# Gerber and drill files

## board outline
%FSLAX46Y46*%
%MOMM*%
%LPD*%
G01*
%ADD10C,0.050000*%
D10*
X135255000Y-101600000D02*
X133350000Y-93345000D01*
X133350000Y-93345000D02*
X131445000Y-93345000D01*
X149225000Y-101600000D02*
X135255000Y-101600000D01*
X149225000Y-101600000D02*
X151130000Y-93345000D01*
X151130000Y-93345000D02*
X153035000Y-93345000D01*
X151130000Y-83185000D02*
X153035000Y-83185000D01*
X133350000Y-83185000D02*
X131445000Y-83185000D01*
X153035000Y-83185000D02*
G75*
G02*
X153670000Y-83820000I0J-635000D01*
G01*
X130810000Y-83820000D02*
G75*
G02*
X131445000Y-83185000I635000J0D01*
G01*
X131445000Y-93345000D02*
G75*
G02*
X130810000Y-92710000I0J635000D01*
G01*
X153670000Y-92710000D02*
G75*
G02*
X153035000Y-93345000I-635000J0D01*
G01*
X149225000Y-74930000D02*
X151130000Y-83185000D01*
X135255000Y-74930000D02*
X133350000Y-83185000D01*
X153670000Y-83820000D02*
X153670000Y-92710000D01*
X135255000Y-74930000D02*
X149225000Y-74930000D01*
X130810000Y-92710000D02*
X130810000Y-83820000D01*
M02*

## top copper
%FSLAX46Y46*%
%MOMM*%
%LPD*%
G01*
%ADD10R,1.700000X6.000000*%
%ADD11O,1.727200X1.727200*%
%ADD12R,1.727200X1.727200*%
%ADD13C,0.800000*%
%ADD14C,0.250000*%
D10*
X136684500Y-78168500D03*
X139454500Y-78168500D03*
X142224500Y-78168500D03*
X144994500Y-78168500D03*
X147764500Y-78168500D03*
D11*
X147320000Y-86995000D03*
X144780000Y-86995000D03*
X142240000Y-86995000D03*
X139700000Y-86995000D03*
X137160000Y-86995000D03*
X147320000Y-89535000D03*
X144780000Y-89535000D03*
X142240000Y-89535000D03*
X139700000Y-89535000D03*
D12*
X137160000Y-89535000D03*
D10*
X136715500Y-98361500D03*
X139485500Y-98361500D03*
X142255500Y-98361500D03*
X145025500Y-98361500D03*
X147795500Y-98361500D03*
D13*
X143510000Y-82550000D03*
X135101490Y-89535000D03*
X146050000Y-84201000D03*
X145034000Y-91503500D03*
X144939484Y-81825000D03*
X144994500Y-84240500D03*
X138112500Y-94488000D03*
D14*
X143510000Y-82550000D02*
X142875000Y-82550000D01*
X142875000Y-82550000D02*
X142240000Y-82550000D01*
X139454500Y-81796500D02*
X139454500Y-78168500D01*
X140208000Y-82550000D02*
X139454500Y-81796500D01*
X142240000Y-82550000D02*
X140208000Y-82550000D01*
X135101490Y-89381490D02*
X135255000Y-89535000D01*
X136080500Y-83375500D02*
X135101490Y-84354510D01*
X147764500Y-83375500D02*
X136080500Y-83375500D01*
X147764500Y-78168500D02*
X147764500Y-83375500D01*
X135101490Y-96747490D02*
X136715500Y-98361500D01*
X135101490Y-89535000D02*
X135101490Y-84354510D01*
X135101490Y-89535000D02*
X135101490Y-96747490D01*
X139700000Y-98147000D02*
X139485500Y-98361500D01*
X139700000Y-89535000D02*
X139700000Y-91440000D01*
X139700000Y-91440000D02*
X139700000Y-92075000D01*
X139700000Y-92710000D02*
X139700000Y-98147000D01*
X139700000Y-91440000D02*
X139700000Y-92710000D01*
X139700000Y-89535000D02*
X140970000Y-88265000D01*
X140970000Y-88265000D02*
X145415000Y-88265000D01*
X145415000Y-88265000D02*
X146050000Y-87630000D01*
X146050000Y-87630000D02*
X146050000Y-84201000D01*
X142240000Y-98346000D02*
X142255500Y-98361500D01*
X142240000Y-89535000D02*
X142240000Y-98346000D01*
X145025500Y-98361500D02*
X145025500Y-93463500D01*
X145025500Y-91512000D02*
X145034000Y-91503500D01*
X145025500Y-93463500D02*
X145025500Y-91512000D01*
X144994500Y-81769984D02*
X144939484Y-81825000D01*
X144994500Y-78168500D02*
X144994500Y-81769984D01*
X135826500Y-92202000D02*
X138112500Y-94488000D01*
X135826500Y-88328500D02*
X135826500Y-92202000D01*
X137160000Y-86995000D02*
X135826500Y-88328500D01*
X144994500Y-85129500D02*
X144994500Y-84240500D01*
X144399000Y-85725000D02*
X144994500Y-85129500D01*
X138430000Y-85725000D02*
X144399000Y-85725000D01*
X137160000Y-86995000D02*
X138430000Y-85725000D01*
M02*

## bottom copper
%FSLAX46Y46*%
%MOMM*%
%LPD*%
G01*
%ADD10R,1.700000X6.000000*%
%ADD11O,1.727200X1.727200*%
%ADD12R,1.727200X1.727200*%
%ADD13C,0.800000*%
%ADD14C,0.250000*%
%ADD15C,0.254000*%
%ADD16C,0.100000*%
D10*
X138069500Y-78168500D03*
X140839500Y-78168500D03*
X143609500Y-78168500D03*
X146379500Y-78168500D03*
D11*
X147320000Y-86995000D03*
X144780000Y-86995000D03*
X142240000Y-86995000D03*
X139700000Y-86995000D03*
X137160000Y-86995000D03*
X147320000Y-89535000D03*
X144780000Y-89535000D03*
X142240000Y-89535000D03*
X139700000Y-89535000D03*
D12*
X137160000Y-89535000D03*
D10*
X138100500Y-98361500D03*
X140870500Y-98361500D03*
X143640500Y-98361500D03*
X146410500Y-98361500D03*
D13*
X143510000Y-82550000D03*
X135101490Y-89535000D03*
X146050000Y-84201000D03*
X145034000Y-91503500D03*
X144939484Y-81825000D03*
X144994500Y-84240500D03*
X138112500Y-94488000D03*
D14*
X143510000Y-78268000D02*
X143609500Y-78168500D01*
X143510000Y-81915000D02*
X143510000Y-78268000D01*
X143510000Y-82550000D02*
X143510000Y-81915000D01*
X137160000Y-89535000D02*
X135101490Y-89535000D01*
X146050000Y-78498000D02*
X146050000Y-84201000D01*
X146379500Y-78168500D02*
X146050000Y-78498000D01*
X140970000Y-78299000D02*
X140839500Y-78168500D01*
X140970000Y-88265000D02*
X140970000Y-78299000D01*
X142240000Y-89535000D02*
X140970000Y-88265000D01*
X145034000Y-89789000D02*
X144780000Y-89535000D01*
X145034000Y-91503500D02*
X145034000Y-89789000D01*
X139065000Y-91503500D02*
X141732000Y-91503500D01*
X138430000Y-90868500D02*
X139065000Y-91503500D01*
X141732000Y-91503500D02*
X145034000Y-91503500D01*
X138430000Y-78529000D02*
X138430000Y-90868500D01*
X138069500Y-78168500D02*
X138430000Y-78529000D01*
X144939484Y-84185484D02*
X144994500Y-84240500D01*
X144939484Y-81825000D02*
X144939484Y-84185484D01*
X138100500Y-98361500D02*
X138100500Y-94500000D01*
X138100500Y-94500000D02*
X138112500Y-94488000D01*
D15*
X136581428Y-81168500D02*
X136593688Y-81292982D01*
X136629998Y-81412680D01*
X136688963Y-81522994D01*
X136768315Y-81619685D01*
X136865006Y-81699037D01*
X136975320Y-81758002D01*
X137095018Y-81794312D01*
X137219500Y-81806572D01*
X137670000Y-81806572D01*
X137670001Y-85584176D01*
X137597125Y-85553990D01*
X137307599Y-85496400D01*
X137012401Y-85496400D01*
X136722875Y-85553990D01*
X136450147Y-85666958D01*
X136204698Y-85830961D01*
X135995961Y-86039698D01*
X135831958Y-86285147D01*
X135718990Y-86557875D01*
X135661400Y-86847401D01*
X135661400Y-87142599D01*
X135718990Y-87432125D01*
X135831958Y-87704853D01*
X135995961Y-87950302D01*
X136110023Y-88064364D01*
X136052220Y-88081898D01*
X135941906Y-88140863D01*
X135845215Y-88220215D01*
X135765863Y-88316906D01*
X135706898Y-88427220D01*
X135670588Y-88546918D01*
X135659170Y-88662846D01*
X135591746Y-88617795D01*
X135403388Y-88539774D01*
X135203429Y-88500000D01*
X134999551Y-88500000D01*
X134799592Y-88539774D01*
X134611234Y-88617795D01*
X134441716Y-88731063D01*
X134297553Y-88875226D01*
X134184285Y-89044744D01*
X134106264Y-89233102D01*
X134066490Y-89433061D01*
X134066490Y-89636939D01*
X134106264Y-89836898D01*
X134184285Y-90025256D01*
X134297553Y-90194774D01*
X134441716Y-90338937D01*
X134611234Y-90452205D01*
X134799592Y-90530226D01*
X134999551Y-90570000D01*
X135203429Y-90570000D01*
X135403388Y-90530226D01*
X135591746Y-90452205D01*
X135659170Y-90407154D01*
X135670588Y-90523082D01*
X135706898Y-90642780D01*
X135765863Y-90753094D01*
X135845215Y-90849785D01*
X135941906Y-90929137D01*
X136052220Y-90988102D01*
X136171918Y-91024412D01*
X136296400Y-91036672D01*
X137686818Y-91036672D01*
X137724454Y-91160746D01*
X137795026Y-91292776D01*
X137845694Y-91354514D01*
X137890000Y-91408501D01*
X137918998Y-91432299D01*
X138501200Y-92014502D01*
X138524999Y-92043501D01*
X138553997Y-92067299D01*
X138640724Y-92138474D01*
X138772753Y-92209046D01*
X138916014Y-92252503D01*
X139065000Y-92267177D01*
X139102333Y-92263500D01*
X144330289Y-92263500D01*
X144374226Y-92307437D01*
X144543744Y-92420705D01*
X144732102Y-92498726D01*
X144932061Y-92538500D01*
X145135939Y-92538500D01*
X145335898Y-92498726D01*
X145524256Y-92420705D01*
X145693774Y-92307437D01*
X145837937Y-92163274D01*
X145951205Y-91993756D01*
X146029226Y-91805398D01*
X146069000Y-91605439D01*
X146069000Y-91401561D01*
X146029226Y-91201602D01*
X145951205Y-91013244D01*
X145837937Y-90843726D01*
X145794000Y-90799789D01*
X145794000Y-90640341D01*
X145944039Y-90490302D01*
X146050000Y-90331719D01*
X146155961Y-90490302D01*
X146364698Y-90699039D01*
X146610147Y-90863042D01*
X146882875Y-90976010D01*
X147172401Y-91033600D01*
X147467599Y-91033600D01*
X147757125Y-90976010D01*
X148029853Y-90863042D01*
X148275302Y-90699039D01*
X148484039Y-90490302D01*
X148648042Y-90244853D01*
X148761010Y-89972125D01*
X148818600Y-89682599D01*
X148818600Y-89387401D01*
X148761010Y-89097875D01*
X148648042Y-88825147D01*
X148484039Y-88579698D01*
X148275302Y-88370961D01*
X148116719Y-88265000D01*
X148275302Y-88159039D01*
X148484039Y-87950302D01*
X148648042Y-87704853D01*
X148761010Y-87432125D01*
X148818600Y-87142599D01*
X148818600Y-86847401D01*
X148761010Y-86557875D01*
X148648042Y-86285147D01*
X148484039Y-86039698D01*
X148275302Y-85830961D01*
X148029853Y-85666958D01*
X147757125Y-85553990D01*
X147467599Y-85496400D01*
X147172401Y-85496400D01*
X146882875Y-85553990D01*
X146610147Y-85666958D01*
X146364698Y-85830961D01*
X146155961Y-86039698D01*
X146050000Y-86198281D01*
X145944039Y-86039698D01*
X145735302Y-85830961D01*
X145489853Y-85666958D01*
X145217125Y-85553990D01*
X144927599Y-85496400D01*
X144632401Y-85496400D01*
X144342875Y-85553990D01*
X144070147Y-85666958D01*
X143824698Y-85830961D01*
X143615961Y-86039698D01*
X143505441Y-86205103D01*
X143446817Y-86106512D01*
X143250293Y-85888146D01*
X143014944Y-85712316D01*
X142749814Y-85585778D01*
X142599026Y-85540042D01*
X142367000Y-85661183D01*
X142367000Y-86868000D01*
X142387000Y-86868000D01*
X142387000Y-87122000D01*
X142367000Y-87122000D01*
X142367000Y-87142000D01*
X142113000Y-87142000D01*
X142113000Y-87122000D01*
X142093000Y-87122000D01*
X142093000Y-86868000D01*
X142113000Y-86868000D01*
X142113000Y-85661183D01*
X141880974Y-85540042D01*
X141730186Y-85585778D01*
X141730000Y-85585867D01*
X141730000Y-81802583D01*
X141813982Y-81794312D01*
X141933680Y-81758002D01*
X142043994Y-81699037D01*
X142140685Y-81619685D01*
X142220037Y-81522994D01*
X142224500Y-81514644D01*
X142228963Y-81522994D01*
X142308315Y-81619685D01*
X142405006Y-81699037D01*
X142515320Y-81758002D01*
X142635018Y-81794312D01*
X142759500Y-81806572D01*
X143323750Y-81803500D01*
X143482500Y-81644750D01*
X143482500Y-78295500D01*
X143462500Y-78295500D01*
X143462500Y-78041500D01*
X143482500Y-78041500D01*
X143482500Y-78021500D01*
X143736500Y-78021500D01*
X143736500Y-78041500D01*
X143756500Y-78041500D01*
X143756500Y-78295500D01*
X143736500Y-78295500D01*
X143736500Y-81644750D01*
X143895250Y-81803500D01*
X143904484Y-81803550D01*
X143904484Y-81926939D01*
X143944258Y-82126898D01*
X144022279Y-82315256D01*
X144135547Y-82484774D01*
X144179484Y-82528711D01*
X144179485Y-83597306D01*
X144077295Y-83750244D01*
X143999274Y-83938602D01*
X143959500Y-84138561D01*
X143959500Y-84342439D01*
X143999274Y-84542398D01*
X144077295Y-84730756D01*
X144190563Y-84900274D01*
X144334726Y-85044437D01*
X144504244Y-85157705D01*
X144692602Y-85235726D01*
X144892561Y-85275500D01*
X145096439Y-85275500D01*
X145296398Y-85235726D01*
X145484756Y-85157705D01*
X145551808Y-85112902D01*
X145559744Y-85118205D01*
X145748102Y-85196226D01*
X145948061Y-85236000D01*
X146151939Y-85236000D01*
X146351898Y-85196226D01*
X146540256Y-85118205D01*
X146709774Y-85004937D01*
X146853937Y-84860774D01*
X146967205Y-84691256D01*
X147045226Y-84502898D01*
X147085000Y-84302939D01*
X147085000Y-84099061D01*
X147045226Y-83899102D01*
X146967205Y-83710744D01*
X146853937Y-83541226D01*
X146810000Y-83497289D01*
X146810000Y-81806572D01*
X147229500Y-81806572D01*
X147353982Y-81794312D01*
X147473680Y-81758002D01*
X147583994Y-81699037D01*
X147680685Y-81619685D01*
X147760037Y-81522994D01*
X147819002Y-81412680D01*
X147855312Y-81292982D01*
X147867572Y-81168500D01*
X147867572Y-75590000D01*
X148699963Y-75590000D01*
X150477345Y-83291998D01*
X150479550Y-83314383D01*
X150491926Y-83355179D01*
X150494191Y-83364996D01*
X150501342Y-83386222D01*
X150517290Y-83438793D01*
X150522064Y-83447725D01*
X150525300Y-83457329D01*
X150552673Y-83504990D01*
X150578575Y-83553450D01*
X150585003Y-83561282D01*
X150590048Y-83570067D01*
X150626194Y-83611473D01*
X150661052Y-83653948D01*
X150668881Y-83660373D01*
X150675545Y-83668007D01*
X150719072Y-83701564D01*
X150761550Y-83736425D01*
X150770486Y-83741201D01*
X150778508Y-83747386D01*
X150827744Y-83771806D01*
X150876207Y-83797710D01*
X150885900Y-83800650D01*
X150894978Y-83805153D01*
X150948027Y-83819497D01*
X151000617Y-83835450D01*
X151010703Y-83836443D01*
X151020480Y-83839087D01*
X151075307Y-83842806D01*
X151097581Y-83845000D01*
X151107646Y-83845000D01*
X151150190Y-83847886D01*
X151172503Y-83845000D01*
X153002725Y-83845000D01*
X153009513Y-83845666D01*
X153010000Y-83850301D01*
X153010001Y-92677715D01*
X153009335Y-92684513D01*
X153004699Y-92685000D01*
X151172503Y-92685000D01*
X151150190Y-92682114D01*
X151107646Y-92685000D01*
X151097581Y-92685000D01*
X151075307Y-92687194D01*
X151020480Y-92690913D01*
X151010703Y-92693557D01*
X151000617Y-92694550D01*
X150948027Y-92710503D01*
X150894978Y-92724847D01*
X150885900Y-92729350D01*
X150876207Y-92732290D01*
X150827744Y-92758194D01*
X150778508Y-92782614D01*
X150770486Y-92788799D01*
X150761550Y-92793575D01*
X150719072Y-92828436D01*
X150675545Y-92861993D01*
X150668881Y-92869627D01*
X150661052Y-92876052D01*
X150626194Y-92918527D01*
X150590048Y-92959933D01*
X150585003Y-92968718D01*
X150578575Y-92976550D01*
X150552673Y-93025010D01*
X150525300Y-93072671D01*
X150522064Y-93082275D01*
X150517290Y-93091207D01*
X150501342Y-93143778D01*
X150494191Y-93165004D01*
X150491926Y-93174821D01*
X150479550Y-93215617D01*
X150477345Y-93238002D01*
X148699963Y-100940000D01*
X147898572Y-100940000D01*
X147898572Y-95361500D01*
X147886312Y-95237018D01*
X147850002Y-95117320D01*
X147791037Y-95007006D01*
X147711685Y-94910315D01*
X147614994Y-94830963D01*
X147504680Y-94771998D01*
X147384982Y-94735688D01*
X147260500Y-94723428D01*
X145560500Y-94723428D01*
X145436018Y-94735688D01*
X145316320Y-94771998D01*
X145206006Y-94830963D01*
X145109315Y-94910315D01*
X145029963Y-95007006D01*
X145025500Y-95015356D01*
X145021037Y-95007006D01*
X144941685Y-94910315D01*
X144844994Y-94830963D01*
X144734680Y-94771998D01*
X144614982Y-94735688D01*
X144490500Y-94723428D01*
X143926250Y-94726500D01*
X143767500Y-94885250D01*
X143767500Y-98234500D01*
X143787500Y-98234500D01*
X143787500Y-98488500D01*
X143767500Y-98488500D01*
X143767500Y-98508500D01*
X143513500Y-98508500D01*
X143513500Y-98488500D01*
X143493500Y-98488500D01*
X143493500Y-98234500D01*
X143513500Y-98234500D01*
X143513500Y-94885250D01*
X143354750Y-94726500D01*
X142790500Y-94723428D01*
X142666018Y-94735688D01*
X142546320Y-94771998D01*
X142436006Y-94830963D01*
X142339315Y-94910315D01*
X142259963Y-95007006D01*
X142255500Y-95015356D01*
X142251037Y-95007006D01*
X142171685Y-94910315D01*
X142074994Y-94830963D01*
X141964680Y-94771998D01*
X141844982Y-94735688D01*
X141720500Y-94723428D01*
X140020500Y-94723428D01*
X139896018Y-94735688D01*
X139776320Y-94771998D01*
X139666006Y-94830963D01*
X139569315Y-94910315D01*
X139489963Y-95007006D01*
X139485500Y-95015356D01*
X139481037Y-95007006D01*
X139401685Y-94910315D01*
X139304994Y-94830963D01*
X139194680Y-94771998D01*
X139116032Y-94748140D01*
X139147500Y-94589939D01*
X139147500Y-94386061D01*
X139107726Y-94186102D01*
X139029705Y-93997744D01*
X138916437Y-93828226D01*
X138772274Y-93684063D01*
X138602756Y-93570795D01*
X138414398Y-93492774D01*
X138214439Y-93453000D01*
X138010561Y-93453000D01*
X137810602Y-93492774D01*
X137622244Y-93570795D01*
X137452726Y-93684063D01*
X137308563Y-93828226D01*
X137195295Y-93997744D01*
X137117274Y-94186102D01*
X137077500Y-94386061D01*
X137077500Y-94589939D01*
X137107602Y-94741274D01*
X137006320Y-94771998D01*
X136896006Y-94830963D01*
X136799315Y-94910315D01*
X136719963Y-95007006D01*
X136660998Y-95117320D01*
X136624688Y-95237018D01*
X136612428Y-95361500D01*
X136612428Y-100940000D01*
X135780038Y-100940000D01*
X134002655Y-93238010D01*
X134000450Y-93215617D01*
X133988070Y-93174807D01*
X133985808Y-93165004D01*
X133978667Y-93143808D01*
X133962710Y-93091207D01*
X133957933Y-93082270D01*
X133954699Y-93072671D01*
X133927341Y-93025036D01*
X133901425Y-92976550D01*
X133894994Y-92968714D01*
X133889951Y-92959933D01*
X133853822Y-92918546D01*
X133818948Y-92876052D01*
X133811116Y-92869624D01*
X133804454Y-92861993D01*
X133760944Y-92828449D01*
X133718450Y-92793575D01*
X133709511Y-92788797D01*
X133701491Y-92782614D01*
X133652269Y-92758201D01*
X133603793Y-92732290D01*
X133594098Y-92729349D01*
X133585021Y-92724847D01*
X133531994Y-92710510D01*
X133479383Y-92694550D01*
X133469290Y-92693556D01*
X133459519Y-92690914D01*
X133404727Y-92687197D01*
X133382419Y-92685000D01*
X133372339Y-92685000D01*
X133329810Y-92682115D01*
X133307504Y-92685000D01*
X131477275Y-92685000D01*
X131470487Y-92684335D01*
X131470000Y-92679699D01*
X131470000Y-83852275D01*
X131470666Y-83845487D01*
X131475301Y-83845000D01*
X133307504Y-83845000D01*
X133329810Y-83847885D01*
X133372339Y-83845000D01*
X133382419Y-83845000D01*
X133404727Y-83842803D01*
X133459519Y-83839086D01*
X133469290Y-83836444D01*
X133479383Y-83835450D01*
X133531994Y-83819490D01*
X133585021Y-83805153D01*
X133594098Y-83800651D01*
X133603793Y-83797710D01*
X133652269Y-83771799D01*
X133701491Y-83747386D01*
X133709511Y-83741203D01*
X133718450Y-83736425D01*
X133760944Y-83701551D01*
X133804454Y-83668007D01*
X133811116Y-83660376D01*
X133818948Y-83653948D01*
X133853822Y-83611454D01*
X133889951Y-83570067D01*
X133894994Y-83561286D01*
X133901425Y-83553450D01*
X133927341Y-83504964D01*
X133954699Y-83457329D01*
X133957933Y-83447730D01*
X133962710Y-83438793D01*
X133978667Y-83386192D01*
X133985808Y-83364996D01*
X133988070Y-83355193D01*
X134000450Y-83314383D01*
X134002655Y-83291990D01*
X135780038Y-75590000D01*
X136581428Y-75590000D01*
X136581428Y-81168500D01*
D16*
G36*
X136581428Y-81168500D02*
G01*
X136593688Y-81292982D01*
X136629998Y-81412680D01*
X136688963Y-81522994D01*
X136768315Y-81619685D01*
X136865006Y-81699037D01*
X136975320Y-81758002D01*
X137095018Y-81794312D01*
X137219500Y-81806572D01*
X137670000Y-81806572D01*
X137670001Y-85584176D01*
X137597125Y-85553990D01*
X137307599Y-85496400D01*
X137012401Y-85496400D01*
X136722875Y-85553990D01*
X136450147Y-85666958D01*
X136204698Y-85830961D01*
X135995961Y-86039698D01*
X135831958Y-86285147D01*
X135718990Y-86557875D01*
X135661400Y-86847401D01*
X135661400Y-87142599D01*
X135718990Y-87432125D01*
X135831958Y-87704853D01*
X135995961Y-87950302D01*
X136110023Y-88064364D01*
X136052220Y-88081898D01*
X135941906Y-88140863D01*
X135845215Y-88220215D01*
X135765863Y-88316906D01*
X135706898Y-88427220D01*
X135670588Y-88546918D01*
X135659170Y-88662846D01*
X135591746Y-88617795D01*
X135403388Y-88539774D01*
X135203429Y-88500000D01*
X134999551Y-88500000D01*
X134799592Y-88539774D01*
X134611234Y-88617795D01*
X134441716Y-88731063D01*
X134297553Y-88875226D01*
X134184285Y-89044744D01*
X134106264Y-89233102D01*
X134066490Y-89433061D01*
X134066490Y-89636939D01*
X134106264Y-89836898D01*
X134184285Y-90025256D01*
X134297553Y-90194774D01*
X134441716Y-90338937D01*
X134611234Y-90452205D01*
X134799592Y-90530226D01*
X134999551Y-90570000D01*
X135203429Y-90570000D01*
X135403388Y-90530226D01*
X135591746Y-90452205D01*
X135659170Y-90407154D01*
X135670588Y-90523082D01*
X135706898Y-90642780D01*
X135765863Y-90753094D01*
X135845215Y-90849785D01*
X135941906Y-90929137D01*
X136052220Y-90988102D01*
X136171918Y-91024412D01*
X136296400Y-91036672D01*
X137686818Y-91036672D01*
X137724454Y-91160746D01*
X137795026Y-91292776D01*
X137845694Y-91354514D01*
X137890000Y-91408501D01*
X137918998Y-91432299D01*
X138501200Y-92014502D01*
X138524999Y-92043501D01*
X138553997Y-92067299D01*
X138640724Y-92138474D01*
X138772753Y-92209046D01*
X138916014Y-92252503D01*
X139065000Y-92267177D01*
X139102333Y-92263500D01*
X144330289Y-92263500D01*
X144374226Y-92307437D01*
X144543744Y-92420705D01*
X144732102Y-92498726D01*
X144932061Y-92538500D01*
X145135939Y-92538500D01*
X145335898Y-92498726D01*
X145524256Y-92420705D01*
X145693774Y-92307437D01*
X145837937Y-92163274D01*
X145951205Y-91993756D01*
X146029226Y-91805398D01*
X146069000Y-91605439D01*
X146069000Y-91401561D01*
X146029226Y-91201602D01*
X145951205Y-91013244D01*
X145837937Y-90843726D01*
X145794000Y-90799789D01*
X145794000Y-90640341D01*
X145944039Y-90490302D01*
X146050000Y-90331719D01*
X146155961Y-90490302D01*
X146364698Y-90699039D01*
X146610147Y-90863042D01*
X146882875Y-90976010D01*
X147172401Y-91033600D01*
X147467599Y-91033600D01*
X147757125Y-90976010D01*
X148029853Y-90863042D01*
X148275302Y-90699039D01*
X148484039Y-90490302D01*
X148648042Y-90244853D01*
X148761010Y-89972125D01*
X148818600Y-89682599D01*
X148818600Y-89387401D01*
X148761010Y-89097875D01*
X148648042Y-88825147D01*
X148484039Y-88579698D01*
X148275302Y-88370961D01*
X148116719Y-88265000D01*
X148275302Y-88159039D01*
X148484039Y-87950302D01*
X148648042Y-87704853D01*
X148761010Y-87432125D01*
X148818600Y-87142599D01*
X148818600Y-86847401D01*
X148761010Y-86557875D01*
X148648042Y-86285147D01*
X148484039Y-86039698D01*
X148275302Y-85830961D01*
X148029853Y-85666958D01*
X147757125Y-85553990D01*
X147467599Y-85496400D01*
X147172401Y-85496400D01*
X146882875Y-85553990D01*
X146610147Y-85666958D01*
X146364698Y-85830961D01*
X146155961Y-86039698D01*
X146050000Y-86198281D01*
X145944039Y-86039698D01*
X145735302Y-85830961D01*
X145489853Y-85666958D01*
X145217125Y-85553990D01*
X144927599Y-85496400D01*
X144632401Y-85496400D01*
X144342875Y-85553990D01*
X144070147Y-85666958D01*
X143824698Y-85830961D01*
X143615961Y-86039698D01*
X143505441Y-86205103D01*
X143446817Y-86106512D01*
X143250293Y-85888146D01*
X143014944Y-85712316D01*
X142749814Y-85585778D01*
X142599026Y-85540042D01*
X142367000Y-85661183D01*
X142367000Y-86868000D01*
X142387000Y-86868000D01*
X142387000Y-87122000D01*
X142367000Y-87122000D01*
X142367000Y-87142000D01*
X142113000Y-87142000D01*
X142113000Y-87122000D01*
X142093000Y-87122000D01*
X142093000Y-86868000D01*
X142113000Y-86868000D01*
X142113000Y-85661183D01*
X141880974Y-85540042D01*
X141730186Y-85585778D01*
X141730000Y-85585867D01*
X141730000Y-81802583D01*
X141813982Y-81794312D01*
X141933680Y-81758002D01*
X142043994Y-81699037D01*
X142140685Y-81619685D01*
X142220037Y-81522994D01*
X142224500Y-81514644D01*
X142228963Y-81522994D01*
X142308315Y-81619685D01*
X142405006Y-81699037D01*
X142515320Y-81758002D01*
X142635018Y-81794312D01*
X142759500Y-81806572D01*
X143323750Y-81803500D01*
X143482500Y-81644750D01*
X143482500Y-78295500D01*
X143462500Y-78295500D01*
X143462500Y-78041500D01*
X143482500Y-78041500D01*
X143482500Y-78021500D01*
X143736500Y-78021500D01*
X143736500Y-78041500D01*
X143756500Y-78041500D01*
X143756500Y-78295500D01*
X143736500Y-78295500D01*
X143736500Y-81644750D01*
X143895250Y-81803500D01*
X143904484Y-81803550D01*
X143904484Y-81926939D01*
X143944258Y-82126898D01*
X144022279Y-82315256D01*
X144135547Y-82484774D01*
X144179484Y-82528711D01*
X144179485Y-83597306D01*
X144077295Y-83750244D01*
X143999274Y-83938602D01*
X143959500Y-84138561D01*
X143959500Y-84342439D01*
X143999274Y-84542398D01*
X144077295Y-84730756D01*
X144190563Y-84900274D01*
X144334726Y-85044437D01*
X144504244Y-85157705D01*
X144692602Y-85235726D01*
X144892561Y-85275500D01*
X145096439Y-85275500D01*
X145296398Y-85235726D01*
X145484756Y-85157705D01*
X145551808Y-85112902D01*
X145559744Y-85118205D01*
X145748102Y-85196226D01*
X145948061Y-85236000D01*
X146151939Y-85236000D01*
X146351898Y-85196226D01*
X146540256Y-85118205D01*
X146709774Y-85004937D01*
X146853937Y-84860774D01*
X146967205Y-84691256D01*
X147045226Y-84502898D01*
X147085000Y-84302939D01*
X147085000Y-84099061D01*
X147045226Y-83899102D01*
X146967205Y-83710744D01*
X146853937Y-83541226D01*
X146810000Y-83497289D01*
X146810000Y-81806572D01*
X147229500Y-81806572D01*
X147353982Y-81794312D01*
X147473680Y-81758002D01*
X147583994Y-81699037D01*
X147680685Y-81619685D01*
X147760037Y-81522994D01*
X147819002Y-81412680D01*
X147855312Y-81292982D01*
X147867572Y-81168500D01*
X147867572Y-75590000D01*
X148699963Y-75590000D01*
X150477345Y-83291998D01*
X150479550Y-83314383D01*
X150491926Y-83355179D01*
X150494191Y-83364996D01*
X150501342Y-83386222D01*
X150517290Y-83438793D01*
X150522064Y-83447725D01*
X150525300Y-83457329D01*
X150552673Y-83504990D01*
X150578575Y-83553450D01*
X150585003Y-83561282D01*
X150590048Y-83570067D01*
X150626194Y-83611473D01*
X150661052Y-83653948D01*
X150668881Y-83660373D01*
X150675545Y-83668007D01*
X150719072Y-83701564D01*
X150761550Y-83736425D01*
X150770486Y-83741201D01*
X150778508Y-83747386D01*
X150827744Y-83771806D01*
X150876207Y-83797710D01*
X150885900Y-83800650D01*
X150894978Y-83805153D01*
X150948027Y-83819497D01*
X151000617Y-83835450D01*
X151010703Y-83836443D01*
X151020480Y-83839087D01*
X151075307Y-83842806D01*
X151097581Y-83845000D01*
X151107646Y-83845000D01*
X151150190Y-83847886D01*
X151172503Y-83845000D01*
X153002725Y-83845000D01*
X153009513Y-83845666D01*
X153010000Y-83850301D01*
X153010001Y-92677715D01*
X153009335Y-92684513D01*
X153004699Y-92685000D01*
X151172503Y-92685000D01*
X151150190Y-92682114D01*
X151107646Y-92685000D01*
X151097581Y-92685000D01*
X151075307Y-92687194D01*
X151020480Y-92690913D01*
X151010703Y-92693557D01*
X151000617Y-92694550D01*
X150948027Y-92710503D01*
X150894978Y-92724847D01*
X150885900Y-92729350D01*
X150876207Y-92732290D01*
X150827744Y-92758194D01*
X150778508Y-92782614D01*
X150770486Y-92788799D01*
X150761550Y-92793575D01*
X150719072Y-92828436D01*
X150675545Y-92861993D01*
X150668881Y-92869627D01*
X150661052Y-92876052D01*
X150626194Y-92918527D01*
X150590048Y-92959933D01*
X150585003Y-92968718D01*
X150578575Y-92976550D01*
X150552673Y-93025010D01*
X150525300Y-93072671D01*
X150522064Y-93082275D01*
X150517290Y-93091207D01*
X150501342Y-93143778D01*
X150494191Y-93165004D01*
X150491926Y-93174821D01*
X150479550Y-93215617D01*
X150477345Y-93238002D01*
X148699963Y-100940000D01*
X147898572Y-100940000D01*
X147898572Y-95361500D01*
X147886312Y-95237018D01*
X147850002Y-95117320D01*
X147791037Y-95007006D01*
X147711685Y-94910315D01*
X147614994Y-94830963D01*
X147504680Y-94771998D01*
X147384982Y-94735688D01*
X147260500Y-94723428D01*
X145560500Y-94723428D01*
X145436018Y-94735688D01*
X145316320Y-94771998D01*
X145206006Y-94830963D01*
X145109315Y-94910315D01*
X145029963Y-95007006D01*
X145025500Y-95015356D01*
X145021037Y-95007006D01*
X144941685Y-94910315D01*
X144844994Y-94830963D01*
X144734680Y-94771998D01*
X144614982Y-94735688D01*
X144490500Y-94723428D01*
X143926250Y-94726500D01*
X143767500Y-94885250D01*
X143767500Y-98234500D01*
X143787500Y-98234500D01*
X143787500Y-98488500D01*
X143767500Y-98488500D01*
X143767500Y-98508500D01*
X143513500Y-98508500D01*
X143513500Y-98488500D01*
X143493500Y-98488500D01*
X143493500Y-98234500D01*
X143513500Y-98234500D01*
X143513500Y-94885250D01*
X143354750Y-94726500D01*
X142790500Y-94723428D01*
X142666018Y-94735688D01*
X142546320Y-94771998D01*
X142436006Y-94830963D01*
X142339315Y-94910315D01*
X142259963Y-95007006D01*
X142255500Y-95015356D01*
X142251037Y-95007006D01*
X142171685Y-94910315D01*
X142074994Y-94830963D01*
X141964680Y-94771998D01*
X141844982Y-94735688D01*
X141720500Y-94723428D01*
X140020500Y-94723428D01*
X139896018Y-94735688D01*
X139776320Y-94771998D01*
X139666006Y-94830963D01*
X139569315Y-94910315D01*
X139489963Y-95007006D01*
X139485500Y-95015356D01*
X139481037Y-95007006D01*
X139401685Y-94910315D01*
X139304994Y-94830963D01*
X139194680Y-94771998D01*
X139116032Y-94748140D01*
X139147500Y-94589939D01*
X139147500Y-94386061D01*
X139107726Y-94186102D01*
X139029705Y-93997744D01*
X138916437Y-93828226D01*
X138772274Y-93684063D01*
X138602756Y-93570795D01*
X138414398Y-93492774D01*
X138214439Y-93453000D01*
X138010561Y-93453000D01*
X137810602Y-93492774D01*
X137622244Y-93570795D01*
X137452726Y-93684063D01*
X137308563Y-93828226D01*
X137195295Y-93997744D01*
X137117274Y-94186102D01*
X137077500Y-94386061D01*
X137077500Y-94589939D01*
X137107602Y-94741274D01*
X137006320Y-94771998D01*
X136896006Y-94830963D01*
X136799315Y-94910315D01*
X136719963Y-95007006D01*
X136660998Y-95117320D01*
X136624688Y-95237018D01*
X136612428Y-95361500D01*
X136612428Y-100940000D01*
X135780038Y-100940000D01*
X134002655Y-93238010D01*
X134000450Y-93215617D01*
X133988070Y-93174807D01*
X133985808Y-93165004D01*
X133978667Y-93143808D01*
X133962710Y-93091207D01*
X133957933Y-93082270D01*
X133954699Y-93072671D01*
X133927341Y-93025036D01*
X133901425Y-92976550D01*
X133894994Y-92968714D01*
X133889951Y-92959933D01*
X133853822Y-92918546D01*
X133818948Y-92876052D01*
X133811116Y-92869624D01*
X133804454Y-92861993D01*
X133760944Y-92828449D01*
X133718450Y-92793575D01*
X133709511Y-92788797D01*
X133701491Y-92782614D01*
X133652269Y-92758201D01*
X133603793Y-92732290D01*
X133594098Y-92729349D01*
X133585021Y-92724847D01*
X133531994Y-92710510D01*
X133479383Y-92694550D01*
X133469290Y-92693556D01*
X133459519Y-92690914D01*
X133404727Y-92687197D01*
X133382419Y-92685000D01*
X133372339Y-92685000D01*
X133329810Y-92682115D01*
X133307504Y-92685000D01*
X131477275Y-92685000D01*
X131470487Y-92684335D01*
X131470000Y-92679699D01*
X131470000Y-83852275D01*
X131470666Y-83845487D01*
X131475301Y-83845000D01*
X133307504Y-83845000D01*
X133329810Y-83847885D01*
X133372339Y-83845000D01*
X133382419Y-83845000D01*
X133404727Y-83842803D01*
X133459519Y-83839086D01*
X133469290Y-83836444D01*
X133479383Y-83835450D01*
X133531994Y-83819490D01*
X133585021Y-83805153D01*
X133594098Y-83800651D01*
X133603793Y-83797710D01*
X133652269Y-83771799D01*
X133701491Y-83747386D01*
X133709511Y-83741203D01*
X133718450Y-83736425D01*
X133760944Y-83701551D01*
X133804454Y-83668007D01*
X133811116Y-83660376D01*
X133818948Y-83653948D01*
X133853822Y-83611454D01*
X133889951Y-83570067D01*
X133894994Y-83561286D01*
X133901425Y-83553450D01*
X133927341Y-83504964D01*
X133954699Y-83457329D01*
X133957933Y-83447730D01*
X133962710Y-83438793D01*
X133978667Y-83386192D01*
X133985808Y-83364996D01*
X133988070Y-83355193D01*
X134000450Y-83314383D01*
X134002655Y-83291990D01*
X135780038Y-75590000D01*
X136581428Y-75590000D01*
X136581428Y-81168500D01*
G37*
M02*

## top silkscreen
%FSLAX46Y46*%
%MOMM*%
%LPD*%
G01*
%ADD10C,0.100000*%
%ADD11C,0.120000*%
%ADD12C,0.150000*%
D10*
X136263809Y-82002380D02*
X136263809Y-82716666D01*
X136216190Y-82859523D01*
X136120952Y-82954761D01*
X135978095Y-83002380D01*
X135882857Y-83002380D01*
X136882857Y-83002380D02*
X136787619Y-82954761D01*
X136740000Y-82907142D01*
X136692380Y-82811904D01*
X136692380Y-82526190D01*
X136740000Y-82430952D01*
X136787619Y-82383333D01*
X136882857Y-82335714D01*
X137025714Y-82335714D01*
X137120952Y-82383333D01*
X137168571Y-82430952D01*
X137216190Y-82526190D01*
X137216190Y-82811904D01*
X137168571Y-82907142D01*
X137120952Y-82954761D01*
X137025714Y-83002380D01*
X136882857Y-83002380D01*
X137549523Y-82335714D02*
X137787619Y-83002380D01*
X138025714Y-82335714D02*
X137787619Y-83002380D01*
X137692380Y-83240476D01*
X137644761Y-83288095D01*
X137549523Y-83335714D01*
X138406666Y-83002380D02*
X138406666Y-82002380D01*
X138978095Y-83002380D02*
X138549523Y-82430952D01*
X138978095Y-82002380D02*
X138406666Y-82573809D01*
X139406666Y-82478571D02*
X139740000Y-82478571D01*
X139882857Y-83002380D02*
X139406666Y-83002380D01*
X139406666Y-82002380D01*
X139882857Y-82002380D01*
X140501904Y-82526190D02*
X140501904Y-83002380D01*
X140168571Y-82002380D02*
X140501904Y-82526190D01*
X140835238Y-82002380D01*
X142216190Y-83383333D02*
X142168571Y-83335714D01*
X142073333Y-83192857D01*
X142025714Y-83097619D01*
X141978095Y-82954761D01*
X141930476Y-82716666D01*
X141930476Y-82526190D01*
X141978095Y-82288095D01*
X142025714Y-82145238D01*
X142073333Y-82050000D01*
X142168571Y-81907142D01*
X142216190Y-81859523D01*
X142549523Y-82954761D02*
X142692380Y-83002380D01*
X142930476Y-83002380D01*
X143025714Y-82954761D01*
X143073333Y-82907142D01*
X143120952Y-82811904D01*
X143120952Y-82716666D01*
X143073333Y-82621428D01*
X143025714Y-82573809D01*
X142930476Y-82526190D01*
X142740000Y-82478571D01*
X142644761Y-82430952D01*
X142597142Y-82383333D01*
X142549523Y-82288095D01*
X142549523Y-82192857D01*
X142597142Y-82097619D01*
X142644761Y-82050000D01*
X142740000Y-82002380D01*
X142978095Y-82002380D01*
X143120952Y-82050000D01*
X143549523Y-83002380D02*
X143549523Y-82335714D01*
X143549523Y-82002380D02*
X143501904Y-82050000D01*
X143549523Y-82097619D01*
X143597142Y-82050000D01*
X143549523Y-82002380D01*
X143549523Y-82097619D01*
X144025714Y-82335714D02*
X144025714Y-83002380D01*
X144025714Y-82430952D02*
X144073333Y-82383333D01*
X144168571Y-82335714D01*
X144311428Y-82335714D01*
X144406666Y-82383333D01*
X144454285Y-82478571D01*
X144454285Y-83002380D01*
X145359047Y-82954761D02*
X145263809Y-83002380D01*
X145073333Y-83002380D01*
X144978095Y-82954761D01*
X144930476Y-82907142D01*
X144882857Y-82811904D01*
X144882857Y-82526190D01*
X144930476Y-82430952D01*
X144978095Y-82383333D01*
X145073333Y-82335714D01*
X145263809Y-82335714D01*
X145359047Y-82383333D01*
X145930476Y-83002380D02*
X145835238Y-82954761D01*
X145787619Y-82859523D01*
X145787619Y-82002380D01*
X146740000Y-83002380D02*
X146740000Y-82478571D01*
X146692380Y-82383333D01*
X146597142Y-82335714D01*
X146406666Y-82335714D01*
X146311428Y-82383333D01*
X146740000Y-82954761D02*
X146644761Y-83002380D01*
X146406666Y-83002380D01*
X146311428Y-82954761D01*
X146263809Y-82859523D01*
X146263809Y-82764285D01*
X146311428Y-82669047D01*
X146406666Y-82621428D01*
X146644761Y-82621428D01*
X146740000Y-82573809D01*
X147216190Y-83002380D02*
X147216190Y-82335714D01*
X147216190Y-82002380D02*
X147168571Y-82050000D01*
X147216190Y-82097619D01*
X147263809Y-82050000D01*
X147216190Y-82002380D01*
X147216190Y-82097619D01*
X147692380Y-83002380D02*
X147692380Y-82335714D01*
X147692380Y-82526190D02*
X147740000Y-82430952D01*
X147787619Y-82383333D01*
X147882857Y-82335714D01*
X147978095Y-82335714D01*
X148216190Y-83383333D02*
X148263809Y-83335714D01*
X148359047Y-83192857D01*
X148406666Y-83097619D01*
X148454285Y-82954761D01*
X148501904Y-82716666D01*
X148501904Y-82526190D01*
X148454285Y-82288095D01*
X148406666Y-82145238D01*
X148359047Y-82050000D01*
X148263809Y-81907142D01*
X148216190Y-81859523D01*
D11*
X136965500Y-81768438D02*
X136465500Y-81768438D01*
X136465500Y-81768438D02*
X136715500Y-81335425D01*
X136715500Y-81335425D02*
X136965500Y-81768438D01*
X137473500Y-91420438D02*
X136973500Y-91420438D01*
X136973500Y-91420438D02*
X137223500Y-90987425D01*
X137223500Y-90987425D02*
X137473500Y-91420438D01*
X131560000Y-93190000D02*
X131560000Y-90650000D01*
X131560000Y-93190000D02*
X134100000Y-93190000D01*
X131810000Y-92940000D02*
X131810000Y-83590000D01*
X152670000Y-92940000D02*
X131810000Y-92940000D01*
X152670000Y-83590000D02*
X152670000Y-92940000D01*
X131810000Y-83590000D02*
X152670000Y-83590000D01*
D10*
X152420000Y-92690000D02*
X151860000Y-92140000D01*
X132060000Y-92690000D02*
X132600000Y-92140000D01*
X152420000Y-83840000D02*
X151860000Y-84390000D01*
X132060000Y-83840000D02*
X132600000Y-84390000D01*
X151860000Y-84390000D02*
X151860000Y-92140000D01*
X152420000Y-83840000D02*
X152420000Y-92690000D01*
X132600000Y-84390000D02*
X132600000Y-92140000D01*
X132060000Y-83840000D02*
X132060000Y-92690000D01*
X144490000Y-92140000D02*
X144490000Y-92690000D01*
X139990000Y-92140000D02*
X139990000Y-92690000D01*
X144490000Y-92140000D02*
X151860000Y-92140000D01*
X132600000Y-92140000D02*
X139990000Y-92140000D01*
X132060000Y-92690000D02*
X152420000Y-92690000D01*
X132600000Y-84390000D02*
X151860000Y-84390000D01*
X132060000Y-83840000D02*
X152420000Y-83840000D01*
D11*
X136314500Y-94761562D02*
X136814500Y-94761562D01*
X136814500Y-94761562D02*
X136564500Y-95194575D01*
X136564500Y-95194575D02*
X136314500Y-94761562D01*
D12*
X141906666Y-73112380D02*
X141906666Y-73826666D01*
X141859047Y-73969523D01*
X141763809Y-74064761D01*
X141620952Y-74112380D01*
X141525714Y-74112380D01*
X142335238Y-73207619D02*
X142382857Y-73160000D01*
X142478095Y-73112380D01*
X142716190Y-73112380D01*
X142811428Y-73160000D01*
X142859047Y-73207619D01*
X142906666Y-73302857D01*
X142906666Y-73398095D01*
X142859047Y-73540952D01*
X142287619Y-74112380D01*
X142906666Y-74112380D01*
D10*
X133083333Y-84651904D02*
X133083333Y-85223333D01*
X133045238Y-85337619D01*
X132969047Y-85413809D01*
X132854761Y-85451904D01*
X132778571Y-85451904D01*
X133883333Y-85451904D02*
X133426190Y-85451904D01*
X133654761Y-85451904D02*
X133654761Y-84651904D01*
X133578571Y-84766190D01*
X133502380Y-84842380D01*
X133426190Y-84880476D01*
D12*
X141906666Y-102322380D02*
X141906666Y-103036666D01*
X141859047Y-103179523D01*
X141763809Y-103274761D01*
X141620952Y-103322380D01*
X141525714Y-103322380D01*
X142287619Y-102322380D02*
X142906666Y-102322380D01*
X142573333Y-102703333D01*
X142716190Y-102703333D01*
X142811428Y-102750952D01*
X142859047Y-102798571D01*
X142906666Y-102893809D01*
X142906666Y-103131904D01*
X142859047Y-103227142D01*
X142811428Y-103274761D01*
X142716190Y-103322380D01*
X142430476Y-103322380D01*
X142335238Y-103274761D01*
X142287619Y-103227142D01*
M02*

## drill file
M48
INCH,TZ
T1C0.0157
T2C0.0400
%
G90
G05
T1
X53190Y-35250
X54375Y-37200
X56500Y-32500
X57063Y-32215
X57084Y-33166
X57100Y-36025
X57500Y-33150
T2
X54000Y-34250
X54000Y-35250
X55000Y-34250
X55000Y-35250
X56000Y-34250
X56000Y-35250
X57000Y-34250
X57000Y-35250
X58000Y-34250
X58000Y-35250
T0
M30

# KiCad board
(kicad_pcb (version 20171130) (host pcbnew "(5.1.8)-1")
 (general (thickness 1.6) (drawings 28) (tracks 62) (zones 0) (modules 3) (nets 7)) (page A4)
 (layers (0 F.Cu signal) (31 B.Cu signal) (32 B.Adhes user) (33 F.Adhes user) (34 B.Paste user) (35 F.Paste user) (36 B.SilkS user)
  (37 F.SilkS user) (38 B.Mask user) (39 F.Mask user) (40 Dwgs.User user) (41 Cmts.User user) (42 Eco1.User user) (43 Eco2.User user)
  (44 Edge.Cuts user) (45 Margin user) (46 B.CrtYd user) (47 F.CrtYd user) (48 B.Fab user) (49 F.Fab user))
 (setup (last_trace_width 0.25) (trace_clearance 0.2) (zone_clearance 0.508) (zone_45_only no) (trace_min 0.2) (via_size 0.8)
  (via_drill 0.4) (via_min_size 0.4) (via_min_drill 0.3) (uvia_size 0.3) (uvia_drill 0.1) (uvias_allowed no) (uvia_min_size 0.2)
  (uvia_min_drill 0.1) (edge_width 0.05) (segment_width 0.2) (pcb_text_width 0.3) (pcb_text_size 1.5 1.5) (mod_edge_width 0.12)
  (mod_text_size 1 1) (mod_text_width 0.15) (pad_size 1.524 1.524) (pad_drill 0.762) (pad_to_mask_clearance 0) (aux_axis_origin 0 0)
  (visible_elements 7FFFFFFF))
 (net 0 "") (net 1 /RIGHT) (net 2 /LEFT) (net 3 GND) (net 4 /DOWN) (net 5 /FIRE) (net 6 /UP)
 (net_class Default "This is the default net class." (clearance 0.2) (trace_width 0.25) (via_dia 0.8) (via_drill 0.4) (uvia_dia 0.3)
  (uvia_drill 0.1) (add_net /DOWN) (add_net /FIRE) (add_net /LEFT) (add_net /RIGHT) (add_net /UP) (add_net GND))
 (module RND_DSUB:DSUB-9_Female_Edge (layer F.Cu) (at 142.24 78.105)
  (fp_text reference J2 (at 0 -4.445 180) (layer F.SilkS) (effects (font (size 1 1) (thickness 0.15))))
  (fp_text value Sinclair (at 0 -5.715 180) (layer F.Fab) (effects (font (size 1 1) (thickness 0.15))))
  (fp_line (start -5.2745 3.663438) (end -5.7745 3.663438) (layer F.SilkS) (width 0.12))
  (fp_line (start -5.7745 3.663438) (end -5.5245 3.230425) (layer F.SilkS) (width 0.12))
  (fp_line (start -5.5245 3.230425) (end -5.2745 3.663438) (layer F.SilkS) (width 0.12))
  (pad 6 smd rect (at -4.1705 0.0635 180) (size 1.7 6) (layers B.Cu B.Paste B.Mask) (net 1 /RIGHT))
  (pad 7 smd rect (at -1.4005 0.0635 180) (size 1.7 6) (layers B.Cu B.Paste B.Mask) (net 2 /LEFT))
  (pad 8 smd rect (at 1.3695 0.0635 180) (size 1.7 6) (layers B.Cu B.Paste B.Mask) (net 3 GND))
  (pad 9 smd rect (at 4.1395 0.0635 180) (size 1.7 6) (layers B.Cu B.Paste B.Mask) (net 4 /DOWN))
  (pad 1 smd rect (at -5.5555 0.0635 180) (size 1.7 6) (layers F.Cu F.Paste F.Mask))
  (pad 2 smd rect (at -2.7855 0.0635 180) (size 1.7 6) (layers F.Cu F.Paste F.Mask) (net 3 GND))
  (pad 3 smd rect (at -0.0155 0.0635 180) (size 1.7 6) (layers F.Cu F.Paste F.Mask))
  (pad 4 smd rect (at 2.7545 0.0635 180) (size 1.7 6) (layers F.Cu F.Paste F.Mask) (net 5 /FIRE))
  (pad 5 smd rect (at 5.5245 0.0635 180) (size 1.7 6) (layers F.Cu F.Paste F.Mask) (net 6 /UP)))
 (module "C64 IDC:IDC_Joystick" (layer F.Cu) (at 137.16 89.535 90)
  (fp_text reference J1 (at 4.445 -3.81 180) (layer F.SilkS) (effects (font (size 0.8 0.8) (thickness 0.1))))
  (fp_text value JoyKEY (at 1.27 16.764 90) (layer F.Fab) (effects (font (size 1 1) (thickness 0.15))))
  (fp_line (start -1.885438 0.3135) (end -1.885438 -0.1865) (layer F.SilkS) (width 0.12))
  (fp_line (start -1.885438 -0.1865) (end -1.452425 0.0635) (layer F.SilkS) (width 0.12))
  (fp_line (start -1.452425 0.0635) (end -1.885438 0.3135) (layer F.SilkS) (width 0.12))
  (fp_line (start -3.655 -5.6) (end -1.115 -5.6) (layer F.SilkS) (width 0.12))
  (fp_line (start -3.655 -5.6) (end -3.655 -3.06) (layer F.SilkS) (width 0.12))
  (fp_line (start -3.405 -5.35) (end 5.945 -5.35) (layer F.SilkS) (width 0.12))
  (fp_line (start -3.405 15.51) (end -3.405 -5.35) (layer F.SilkS) (width 0.12))
  (fp_line (start 5.945 15.51) (end -3.405 15.51) (layer F.SilkS) (width 0.12))
  (fp_line (start 5.945 -5.35) (end 5.945 15.51) (layer F.SilkS) (width 0.12))
  (fp_line (start -3.155 15.26) (end -2.605 14.7) (layer F.SilkS) (width 0.1))
  (fp_line (start -3.155 -5.1) (end -2.605 -4.56) (layer F.SilkS) (width 0.1))
  (fp_line (start 5.695 15.26) (end 5.145 14.7) (layer F.SilkS) (width 0.1))
  (fp_line (start 5.695 -5.1) (end 5.145 -4.56) (layer F.SilkS) (width 0.1))
  (fp_line (start 5.145 14.7) (end -2.605 14.7) (layer F.SilkS) (width 0.1))
  (fp_line (start 5.695 15.26) (end -3.155 15.26) (layer F.SilkS) (width 0.1))
  (fp_line (start 5.145 -4.56) (end -2.605 -4.56) (layer F.SilkS) (width 0.1))
  (fp_line (start 5.695 -5.1) (end -3.155 -5.1) (layer F.SilkS) (width 0.1))
  (fp_line (start -2.605 7.33) (end -3.155 7.33) (layer F.SilkS) (width 0.1))
  (fp_line (start -2.605 2.83) (end -3.155 2.83) (layer F.SilkS) (width 0.1))
  (fp_line (start -2.605 7.33) (end -2.605 14.7) (layer F.SilkS) (width 0.1))
  (fp_line (start -2.605 -4.56) (end -2.605 2.83) (layer F.SilkS) (width 0.1))
  (fp_line (start -3.155 -5.1) (end -3.155 15.26) (layer F.SilkS) (width 0.1))
  (fp_line (start 5.145 -4.56) (end 5.145 14.7) (layer F.SilkS) (width 0.1))
  (fp_line (start 5.695 -5.1) (end 5.695 15.26) (layer F.SilkS) (width 0.1))
  (pad 10 thru_hole oval (at 2.54 10.16 90) (size 1.7272 1.7272) (drill 1.016) (layers *.Cu *.Mask))
  (pad 9 thru_hole oval (at 2.54 7.62 90) (size 1.7272 1.7272) (drill 1.016) (layers *.Cu *.Mask))
  (pad 8 thru_hole oval (at 2.54 5.08 90) (size 1.7272 1.7272) (drill 1.016) (layers *.Cu *.Mask) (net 3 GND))
  (pad 7 thru_hole oval (at 2.54 2.54 90) (size 1.7272 1.7272) (drill 1.016) (layers *.Cu *.Mask))
  (pad 6 thru_hole oval (at 2.54 0 90) (size 1.7272 1.7272) (drill 1.016) (layers *.Cu *.Mask) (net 5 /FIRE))
  (pad 5 thru_hole oval (at 0 10.16 90) (size 1.7272 1.7272) (drill 1.016) (layers *.Cu *.Mask))
  (pad 4 thru_hole oval (at 0 7.62 90) (size 1.7272 1.7272) (drill 1.016) (layers *.Cu *.Mask) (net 1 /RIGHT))
  (pad 3 thru_hole oval (at 0 5.08 90) (size 1.7272 1.7272) (drill 1.016) (layers *.Cu *.Mask) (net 2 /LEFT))
  (pad 2 thru_hole oval (at 0 2.54 90) (size 1.7272 1.7272) (drill 1.016) (layers *.Cu *.Mask) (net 4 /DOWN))
  (pad 1 thru_hole rect (at 0 0 90) (size 1.7272 1.7272) (drill 1.016) (layers *.Cu *.Mask) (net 6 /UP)))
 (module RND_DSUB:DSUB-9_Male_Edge (layer F.Cu) (at 142.24 98.425 180)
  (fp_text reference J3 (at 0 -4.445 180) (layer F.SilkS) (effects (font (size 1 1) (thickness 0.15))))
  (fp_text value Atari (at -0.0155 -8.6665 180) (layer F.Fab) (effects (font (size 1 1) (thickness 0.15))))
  (fp_line (start 5.9255 3.663438) (end 5.4255 3.663438) (layer F.SilkS) (width 0.12))
  (fp_line (start 5.4255 3.663438) (end 5.6755 3.230425) (layer F.SilkS) (width 0.12))
  (fp_line (start 5.6755 3.230425) (end 5.9255 3.663438) (layer F.SilkS) (width 0.12))
  (pad 1 smd rect (at 5.5245 0.0635) (size 1.7 6) (layers F.Cu F.Paste F.Mask) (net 6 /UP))
  (pad 2 smd rect (at 2.7545 0.0635) (size 1.7 6) (layers F.Cu F.Paste F.Mask) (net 4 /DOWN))
  (pad 3 smd rect (at -0.0155 0.0635) (size 1.7 6) (layers F.Cu F.Paste F.Mask) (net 2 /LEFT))
  (pad 4 smd rect (at -2.7855 0.0635) (size 1.7 6) (layers F.Cu F.Paste F.Mask) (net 1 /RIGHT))
  (pad 5 smd rect (at -5.5555 0.0635) (size 1.7 6) (layers F.Cu F.Paste F.Mask))
  (pad 6 smd rect (at 4.1395 0.0635) (size 1.7 6) (layers B.Cu B.Paste B.Mask) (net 5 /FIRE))
  (pad 7 smd rect (at 1.3695 0.0635) (size 1.7 6) (layers B.Cu B.Paste B.Mask))
  (pad 8 smd rect (at -1.4005 0.0635) (size 1.7 6) (layers B.Cu B.Paste B.Mask) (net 3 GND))
  (pad 9 smd rect (at -4.1705 0.0635) (size 1.7 6) (layers B.Cu B.Paste B.Mask)))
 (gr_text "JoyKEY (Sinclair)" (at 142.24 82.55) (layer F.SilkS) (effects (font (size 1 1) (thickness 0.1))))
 (gr_line (start 135.255 101.6) (end 133.35 93.345) (layer Edge.Cuts) (width 0.05))
 (gr_line (start 133.35 93.345) (end 131.445 93.345) (layer Edge.Cuts) (width 0.05))
 (gr_line (start 149.225 101.6) (end 135.255 101.6) (layer Edge.Cuts) (width 0.05))
 (gr_line (start 149.225 101.6) (end 151.13 93.345) (layer Edge.Cuts) (width 0.05))
 (gr_line (start 151.13 93.345) (end 153.035 93.345) (layer Edge.Cuts) (width 0.05))
 (gr_line (start 151.13 83.185) (end 153.035 83.185) (layer Edge.Cuts) (width 0.05))
 (gr_line (start 133.35 83.185) (end 131.445 83.185) (layer Edge.Cuts) (width 0.05))
 (gr_arc (start 153.035 83.82) (end 153.67 83.82) (angle -90) (layer Edge.Cuts) (width 0.05))
 (gr_arc (start 131.445 83.82) (end 131.445 83.185) (angle -90) (layer Edge.Cuts) (width 0.05))
 (gr_arc (start 131.445 92.71) (end 130.81 92.71) (angle -90) (layer Edge.Cuts) (width 0.05))
 (gr_arc (start 153.035 92.71) (end 153.035 93.345) (angle -90) (layer Edge.Cuts) (width 0.05))
 (gr_line (start 149.225 74.93) (end 151.13 83.185) (layer Edge.Cuts) (width 0.05))
 (gr_line (start 135.255 74.93) (end 133.35 83.185) (layer Edge.Cuts) (width 0.05))
 (gr_line (start 153.67 83.82) (end 153.67 92.71) (layer Edge.Cuts) (width 0.05))
 (gr_line (start 135.255 74.93) (end 149.225 74.93) (layer Edge.Cuts) (width 0.05))
 (gr_line (start 130.81 92.71) (end 130.81 83.82) (layer Edge.Cuts) (width 0.05))
 (segment (start 143.51 78.268) (end 143.6095 78.1685) (width 0.25) (layer B.Cu) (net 3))
 (segment (start 143.51 81.915) (end 143.51 78.268) (width 0.25) (layer B.Cu) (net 3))
 (via (at 143.51 82.55) (size 0.8) (drill 0.4) (layers F.Cu B.Cu) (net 3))
 (segment (start 143.51 82.55) (end 143.51 81.915) (width 0.25) (layer B.Cu) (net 3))
 (segment (start 143.51 82.55) (end 142.875 82.55) (width 0.25) (layer F.Cu) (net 3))
 (segment (start 142.875 82.55) (end 142.24 82.55) (width 0.25) (layer F.Cu) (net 3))
 (segment (start 139.4545 81.7965) (end 139.4545 78.1685) (width 0.25) (layer F.Cu) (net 3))
 (segment (start 140.208 82.55) (end 139.4545 81.7965) (width 0.25) (layer F.Cu) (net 3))
 (segment (start 142.24 82.55) (end 140.208 82.55) (width 0.25) (layer F.Cu) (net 3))
 (via (at 135.10149 89.535) (size 0.8) (drill 0.4) (layers F.Cu B.Cu) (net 6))
 (segment (start 137.16 89.535) (end 135.10149 89.535) (width 0.25) (layer B.Cu) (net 6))
 (segment (start 135.10149 89.38149) (end 135.255 89.535) (width 0.25) (layer F.Cu) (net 6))
 (segment (start 136.0805 83.3755) (end 135.10149 84.35451) (width 0.25) (layer F.Cu) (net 6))
 (segment (start 147.7645 83.3755) (end 136.0805 83.3755) (width 0.25) (layer F.Cu) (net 6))
 (segment (start 147.7645 78.1685) (end 147.7645 83.3755) (width 0.25) (layer F.Cu) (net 6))
 (segment (start 135.10149 96.74749) (end 136.7155 98.3615) (width 0.25) (layer F.Cu) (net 6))
 (segment (start 135.10149 89.535) (end 135.10149 84.35451) (width 0.25) (layer F.Cu) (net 6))
 (segment (start 135.10149 89.535) (end 135.10149 96.74749) (width 0.25) (layer F.Cu) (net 6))
 (via (at 146.05 84.201) (size 0.8) (drill 0.4) (layers F.Cu B.Cu) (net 4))
 (segment (start 146.05 78.498) (end 146.05 84.201) (width 0.25) (layer B.Cu) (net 4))
 (segment (start 146.3795 78.1685) (end 146.05 78.498) (width 0.25) (layer B.Cu) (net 4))
 (segment (start 139.7 98.147) (end 139.4855 98.3615) (width 0.25) (layer F.Cu) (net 4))
 (segment (start 139.7 89.535) (end 139.7 91.44) (width 0.25) (layer F.Cu) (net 4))
 (segment (start 139.7 91.44) (end 139.7 92.075) (width 0.25) (layer F.Cu) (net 4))
 (segment (start 139.7 92.71) (end 139.7 98.147) (width 0.25) (layer F.Cu) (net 4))
 (segment (start 139.7 91.44) (end 139.7 92.71) (width 0.25) (layer F.Cu) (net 4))
 (segment (start 139.7 89.535) (end 140.97 88.265) (width 0.25) (layer F.Cu) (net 4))
 (segment (start 140.97 88.265) (end 145.415 88.265) (width 0.25) (layer F.Cu) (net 4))
 (segment (start 145.415 88.265) (end 146.05 87.63) (width 0.25) (layer F.Cu) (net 4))
 (segment (start 146.05 87.63) (end 146.05 84.201) (width 0.25) (layer F.Cu) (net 4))
 (segment (start 142.24 98.346) (end 142.2555 98.3615) (width 0.25) (layer F.Cu) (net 2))
 (segment (start 142.24 89.535) (end 142.24 98.346) (width 0.25) (layer F.Cu) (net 2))
 (segment (start 140.97 78.299) (end 140.8395 78.1685) (width 0.25) (layer B.Cu) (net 2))
 (segment (start 140.97 88.265) (end 140.97 78.299) (width 0.25) (layer B.Cu) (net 2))
 (segment (start 142.24 89.535) (end 140.97 88.265) (width 0.25) (layer B.Cu) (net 2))
 (segment (start 145.0255 98.3615) (end 145.0255 93.4635) (width 0.25) (layer F.Cu) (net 1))
 (via (at 145.034 91.5035) (size 0.8) (drill 0.4) (layers F.Cu B.Cu) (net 1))
 (segment (start 145.0255 91.512) (end 145.034 91.5035) (width 0.25) (layer F.Cu) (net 1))
 (segment (start 145.0255 93.4635) (end 145.0255 91.512) (width 0.25) (layer F.Cu) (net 1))
 (segment (start 145.034 89.789) (end 144.78 89.535) (width 0.25) (layer B.Cu) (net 1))
 (segment (start 145.034 91.5035) (end 145.034 89.789) (width 0.25) (layer B.Cu) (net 1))
 (segment (start 139.065 91.5035) (end 141.732 91.5035) (width 0.25) (layer B.Cu) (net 1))
 (segment (start 138.43 90.8685) (end 139.065 91.5035) (width 0.25) (layer B.Cu) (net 1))
 (segment (start 141.732 91.5035) (end 145.034 91.5035) (width 0.25) (layer B.Cu) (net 1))
 (segment (start 138.43 78.529) (end 138.43 90.8685) (width 0.25) (layer B.Cu) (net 1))
 (segment (start 138.0695 78.1685) (end 138.43 78.529) (width 0.25) (layer B.Cu) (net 1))
 (via (at 144.939484 81.825) (size 0.8) (drill 0.4) (layers F.Cu B.Cu) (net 5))
 (segment (start 144.9945 81.769984) (end 144.939484 81.825) (width 0.25) (layer F.Cu) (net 5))
 (segment (start 144.9945 78.1685) (end 144.9945 81.769984) (width 0.25) (layer F.Cu) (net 5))
 (via (at 144.9945 84.2405) (size 0.8) (drill 0.4) (layers F.Cu B.Cu) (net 5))
 (segment (start 144.939484 84.185484) (end 144.9945 84.2405) (width 0.25) (layer B.Cu) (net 5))
 (segment (start 144.939484 81.825) (end 144.939484 84.185484) (width 0.25) (layer B.Cu) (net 5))
 (via (at 138.1125 94.488) (size 0.8) (drill 0.4) (layers F.Cu B.Cu) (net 5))
 (segment (start 138.1005 98.3615) (end 138.1005 94.5) (width 0.25) (layer B.Cu) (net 5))
 (segment (start 138.1005 94.5) (end 138.1125 94.488) (width 0.25) (layer B.Cu) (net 5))
 (segment (start 135.8265 92.202) (end 138.1125 94.488) (width 0.25) (layer F.Cu) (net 5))
 (segment (start 135.8265 88.3285) (end 135.8265 92.202) (width 0.25) (layer F.Cu) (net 5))
 (segment (start 137.16 86.995) (end 135.8265 88.3285) (width 0.25) (layer F.Cu) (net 5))
 (segment (start 144.9945 85.1295) (end 144.9945 84.2405) (width 0.25) (layer F.Cu) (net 5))
 (segment (start 144.399 85.725) (end 144.9945 85.1295) (width 0.25) (layer F.Cu) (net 5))
 (segment (start 138.43 85.725) (end 144.399 85.725) (width 0.25) (layer F.Cu) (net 5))
 (segment (start 137.16 86.995) (end 138.43 85.725) (width 0.25) (layer F.Cu) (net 5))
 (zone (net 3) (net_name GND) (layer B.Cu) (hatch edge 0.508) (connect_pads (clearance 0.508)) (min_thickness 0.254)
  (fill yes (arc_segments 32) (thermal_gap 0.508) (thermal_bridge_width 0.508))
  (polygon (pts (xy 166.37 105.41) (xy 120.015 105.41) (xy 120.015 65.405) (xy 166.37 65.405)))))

